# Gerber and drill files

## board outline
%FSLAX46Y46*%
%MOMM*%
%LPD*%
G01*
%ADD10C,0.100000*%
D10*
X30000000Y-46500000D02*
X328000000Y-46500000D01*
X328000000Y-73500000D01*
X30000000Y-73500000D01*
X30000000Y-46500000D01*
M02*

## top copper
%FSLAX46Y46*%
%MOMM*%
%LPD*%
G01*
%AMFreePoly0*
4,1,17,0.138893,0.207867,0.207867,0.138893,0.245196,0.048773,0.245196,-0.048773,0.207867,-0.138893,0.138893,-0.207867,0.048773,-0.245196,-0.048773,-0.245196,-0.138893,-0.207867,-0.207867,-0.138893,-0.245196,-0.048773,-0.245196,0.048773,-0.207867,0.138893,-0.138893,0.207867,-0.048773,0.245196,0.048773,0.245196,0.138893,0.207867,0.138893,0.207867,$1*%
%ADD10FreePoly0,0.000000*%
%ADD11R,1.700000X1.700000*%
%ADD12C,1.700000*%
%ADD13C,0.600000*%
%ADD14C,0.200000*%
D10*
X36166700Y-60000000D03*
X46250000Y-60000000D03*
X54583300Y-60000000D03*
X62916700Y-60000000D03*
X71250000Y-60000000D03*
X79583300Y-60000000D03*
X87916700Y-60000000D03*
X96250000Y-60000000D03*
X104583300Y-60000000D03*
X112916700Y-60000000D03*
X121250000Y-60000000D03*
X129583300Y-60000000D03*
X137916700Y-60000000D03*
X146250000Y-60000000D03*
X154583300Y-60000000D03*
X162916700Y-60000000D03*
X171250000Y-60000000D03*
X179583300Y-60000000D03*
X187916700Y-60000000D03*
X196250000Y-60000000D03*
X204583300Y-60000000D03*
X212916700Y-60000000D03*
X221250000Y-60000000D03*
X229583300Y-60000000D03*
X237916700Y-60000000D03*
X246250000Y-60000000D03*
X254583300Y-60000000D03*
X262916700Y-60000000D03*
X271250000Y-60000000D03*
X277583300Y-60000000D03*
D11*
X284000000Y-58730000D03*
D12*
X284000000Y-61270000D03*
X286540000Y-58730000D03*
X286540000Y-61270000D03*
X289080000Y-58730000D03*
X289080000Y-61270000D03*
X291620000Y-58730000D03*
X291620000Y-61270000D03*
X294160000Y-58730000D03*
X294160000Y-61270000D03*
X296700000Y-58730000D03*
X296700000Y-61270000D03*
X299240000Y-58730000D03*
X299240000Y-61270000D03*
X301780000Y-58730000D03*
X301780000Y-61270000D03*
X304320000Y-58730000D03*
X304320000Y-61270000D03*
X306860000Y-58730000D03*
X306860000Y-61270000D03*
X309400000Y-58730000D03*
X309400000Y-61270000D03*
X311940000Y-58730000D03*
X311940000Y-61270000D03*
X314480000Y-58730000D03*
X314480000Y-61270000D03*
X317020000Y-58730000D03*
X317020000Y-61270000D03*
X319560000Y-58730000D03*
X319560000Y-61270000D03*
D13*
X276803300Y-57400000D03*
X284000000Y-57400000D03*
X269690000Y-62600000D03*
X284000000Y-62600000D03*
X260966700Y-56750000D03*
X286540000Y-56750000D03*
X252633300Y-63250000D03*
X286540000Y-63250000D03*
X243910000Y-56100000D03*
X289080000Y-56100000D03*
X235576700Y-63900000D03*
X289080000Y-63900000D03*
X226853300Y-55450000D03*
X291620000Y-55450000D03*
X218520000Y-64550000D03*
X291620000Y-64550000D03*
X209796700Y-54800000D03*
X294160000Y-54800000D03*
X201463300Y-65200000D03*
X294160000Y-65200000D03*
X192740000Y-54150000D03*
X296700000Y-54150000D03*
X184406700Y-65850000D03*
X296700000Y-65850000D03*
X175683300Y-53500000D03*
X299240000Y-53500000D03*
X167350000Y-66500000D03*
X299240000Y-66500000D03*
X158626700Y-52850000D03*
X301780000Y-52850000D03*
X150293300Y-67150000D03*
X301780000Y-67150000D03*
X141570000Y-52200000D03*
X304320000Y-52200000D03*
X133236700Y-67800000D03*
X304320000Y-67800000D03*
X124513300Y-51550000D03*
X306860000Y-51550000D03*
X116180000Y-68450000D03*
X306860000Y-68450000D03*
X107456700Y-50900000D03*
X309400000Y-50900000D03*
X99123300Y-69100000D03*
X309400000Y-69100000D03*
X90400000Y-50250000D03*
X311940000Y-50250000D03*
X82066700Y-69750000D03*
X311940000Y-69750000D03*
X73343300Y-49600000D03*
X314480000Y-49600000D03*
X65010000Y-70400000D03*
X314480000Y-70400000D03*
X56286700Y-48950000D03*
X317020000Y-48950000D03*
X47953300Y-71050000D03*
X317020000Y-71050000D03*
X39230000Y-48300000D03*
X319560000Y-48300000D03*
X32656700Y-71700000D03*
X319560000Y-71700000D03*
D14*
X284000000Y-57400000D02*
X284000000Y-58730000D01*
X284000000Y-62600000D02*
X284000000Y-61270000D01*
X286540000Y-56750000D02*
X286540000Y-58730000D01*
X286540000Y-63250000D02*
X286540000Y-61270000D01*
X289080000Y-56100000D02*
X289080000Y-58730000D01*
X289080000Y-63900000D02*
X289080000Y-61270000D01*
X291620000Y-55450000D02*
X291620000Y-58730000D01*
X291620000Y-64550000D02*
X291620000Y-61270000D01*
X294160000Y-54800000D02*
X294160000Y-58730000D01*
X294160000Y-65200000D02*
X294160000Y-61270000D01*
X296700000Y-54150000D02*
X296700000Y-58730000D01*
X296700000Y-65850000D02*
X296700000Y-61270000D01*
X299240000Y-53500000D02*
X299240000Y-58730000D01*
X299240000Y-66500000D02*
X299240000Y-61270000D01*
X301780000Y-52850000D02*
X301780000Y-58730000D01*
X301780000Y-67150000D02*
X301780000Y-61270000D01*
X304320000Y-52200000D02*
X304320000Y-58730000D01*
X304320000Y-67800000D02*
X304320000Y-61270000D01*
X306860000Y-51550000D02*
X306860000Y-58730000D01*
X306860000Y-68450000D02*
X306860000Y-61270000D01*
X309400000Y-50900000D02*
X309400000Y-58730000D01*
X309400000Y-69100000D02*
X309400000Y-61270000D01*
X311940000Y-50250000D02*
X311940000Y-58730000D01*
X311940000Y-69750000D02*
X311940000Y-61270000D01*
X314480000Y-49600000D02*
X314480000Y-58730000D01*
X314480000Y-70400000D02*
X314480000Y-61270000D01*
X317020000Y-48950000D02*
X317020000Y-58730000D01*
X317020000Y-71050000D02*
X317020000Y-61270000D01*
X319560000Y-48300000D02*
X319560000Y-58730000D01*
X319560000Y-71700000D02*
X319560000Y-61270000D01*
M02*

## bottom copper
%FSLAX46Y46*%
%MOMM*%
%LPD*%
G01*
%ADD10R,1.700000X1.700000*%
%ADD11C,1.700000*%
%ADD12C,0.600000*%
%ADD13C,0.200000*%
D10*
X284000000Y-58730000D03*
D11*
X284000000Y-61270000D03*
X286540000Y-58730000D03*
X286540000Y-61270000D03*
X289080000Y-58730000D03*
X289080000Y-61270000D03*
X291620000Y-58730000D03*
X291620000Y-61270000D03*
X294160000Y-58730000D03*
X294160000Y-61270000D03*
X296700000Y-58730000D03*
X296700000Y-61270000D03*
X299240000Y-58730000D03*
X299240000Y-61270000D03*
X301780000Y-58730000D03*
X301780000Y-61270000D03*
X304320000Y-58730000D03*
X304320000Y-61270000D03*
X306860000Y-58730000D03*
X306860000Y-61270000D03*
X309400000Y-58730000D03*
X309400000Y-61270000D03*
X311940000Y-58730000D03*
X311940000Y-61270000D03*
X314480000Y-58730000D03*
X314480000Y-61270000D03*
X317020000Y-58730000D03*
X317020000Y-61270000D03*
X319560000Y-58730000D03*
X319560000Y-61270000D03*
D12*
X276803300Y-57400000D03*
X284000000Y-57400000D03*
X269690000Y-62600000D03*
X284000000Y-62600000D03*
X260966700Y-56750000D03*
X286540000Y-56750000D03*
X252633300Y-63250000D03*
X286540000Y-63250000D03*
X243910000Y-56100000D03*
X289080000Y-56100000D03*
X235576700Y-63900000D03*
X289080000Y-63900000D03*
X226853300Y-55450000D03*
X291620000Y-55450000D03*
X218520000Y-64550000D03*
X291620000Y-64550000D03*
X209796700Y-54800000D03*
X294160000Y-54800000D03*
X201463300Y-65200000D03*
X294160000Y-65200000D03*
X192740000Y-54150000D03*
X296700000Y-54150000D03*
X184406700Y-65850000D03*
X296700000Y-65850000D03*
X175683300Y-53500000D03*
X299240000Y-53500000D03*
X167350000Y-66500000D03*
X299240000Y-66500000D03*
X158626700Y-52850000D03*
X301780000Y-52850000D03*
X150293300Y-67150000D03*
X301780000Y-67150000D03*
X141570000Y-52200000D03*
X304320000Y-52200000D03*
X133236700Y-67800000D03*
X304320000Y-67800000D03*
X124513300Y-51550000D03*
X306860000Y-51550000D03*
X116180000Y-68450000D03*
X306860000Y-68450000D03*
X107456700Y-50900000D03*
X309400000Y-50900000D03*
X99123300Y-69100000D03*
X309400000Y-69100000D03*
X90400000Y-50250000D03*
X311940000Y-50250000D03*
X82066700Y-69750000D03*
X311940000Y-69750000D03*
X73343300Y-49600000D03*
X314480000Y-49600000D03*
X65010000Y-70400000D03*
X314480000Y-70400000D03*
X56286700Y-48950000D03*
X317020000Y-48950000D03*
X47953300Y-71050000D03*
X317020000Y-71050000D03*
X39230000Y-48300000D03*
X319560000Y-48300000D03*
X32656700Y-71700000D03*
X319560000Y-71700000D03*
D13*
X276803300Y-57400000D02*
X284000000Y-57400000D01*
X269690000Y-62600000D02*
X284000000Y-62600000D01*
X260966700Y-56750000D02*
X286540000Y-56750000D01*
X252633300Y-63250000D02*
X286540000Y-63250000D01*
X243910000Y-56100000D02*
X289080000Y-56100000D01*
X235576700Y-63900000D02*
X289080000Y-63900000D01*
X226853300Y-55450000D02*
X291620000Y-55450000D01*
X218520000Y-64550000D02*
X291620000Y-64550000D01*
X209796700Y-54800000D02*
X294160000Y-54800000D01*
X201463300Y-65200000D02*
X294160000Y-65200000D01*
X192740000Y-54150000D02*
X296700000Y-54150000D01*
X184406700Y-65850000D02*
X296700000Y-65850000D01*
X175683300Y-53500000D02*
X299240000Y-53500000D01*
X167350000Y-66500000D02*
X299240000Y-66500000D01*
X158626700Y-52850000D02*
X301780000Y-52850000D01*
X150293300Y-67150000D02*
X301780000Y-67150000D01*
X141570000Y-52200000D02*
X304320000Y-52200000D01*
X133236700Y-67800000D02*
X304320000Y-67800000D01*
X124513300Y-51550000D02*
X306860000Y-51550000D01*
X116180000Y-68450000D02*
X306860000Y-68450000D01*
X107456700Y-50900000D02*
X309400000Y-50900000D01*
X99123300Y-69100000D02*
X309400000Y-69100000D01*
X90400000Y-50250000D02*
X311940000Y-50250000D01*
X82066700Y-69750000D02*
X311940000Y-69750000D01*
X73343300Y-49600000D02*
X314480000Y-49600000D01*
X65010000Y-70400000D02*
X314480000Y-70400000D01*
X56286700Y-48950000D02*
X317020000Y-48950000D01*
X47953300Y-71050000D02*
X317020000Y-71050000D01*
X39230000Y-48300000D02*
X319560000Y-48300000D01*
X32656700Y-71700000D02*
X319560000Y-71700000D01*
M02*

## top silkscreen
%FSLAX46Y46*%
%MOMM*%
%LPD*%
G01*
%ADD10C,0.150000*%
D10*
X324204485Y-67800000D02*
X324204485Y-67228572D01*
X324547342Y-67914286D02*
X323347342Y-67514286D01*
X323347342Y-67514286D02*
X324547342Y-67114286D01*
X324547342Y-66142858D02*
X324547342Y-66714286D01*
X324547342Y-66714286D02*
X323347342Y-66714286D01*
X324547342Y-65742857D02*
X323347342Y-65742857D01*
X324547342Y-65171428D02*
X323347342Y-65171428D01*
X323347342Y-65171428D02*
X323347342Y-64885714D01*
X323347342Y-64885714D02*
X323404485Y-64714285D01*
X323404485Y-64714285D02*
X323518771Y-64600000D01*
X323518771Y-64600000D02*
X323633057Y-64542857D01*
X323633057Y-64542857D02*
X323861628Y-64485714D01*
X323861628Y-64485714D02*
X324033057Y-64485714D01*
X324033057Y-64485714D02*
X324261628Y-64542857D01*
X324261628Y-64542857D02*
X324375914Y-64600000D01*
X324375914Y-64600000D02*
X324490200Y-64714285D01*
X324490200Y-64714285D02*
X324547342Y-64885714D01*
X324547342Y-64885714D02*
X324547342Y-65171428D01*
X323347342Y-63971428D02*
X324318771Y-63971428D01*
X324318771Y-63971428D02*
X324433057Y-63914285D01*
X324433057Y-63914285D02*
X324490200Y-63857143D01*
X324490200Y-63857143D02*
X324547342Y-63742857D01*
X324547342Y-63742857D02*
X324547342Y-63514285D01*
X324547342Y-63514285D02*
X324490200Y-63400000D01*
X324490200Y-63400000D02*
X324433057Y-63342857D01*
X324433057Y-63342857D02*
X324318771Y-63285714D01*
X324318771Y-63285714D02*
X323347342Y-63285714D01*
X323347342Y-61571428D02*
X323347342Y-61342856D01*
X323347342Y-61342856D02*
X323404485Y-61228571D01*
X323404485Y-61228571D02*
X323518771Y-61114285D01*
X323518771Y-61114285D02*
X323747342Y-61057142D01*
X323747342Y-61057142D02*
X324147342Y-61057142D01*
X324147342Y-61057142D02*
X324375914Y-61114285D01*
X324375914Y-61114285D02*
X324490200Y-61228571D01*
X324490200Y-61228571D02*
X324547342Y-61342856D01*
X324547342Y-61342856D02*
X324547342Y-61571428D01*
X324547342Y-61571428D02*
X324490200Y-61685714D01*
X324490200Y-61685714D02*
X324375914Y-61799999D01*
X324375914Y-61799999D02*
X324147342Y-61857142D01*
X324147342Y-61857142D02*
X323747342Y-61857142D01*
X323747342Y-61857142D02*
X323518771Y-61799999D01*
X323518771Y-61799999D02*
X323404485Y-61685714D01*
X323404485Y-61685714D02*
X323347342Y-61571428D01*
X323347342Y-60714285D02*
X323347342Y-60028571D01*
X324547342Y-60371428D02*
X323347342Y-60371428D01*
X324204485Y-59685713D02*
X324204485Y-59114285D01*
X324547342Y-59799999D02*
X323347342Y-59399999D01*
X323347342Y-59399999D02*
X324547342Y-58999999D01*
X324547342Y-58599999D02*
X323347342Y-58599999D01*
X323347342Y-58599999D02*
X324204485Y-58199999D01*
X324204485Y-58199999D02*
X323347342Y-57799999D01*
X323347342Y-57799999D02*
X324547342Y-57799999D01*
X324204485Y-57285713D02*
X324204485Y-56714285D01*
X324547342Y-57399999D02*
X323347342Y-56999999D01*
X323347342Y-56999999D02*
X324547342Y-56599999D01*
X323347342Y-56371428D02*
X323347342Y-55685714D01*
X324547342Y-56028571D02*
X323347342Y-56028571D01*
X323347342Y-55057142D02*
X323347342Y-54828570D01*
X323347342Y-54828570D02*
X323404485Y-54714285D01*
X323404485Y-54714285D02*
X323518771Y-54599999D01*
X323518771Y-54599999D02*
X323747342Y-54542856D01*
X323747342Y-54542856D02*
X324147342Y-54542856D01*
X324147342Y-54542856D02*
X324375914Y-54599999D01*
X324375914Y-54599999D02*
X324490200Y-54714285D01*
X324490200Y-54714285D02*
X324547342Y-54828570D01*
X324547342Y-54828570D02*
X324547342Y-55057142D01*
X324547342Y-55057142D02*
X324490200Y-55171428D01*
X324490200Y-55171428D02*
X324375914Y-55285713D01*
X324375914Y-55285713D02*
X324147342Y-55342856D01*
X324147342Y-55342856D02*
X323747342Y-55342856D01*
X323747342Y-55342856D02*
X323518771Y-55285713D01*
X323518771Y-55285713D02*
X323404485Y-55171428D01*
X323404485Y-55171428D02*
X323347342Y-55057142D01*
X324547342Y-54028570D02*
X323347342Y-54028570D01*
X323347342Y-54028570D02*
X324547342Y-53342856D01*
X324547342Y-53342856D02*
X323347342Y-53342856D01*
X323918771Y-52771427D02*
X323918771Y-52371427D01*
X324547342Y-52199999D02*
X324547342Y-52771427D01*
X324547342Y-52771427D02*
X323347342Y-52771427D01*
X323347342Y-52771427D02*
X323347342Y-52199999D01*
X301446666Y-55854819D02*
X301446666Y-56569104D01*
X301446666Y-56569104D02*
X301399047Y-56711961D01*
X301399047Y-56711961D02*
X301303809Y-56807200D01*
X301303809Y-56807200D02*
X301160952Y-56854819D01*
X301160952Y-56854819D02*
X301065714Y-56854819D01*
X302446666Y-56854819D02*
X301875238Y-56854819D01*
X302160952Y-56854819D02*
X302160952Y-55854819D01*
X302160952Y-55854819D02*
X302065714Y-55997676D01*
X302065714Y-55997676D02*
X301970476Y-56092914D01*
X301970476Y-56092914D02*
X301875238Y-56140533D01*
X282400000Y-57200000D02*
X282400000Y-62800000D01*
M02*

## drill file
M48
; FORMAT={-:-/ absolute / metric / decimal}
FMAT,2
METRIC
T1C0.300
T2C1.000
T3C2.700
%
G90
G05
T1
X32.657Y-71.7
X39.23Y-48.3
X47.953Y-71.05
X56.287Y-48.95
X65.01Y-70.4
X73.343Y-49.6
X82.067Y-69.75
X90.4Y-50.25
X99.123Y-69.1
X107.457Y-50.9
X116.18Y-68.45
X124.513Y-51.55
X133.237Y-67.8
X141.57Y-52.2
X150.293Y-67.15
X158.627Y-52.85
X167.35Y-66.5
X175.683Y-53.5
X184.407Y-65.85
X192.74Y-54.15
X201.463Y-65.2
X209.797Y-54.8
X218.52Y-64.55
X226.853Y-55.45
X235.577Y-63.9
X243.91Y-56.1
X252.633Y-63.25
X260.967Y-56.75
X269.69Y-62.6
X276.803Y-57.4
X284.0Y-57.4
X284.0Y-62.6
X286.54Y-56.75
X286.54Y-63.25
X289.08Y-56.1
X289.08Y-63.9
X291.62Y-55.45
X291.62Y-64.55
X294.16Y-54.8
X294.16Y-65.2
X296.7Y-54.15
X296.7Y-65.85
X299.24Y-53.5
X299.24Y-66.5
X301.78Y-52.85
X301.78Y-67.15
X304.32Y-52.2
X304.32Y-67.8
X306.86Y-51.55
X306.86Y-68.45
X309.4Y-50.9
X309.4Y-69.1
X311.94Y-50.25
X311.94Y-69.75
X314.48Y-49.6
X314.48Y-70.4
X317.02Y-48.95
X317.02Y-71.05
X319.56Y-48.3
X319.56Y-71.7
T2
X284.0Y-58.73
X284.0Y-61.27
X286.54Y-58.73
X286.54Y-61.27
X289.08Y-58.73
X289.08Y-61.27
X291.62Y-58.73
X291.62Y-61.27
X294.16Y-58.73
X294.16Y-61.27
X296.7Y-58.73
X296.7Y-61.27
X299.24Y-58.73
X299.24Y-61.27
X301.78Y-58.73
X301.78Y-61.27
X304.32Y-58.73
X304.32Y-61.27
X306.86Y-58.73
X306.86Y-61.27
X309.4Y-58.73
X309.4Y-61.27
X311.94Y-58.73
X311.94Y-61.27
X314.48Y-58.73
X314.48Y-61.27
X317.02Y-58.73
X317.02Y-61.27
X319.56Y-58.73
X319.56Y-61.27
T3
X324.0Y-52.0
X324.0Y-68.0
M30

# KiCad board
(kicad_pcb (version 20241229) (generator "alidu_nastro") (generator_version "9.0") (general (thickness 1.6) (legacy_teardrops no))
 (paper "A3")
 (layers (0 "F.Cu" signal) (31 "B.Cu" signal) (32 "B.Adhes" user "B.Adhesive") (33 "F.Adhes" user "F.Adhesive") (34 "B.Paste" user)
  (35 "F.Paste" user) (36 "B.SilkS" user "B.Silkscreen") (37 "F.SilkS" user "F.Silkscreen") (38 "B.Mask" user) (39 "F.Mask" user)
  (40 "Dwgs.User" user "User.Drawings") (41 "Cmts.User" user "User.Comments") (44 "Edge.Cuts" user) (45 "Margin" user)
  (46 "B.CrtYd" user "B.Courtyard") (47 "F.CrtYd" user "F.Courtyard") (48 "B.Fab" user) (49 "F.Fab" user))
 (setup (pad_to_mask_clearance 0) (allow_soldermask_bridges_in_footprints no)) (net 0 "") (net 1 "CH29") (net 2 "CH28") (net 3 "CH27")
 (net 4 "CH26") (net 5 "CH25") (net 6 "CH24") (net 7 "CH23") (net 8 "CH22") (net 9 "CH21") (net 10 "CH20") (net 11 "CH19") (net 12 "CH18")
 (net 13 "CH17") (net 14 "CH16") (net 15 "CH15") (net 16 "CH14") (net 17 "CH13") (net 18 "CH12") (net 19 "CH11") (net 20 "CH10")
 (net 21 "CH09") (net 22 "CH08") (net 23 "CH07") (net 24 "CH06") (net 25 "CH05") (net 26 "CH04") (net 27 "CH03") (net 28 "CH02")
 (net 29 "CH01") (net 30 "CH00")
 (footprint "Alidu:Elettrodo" (layer "F.Cu") (at 36.1667 60.0)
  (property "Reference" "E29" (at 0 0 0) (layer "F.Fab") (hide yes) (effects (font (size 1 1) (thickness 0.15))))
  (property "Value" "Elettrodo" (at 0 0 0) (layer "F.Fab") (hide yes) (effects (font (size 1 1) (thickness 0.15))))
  (pad "1" smd custom (at 0 0) (size 0.5 0.5) (layers "F.Cu") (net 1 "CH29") (zone_connect 0) (options (clearance outline) (anchor circle))
   (primitives)))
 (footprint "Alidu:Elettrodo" (layer "F.Cu") (at 46.25 60.0)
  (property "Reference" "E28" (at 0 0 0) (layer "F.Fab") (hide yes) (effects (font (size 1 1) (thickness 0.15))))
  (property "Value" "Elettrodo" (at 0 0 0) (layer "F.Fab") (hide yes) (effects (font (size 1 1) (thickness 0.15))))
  (pad "1" smd custom (at 0 0) (size 0.5 0.5) (layers "F.Cu") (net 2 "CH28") (zone_connect 0) (options (clearance outline) (anchor circle))
   (primitives)))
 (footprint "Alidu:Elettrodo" (layer "F.Cu") (at 54.5833 60.0)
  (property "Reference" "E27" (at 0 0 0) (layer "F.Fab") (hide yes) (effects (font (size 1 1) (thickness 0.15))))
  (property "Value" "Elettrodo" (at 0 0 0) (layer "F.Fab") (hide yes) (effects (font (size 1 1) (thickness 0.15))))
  (pad "1" smd custom (at 0 0) (size 0.5 0.5) (layers "F.Cu") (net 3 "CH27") (zone_connect 0) (options (clearance outline) (anchor circle))
   (primitives)))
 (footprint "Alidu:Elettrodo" (layer "F.Cu") (at 62.9167 60.0)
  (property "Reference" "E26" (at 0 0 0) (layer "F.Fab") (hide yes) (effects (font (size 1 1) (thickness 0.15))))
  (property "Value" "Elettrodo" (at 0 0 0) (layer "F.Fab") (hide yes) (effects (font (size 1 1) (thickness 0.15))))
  (pad "1" smd custom (at 0 0) (size 0.5 0.5) (layers "F.Cu") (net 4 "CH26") (zone_connect 0) (options (clearance outline) (anchor circle))
   (primitives)))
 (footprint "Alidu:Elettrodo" (layer "F.Cu") (at 71.25 60.0)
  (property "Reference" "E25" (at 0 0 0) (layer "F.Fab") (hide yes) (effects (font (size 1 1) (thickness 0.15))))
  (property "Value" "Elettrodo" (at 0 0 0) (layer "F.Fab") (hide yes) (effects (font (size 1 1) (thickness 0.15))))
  (pad "1" smd custom (at 0 0) (size 0.5 0.5) (layers "F.Cu") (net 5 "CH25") (zone_connect 0) (options (clearance outline) (anchor circle))
   (primitives)))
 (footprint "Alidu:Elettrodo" (layer "F.Cu") (at 79.5833 60.0)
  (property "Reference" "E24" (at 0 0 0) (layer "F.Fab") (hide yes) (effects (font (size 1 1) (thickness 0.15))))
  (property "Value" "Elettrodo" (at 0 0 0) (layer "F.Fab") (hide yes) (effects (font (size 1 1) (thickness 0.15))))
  (pad "1" smd custom (at 0 0) (size 0.5 0.5) (layers "F.Cu") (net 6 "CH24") (zone_connect 0) (options (clearance outline) (anchor circle))
   (primitives)))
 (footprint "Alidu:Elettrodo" (layer "F.Cu") (at 87.9167 60.0)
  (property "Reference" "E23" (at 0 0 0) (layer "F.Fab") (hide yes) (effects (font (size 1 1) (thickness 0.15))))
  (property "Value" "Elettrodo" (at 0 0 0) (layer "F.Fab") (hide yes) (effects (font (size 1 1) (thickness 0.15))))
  (pad "1" smd custom (at 0 0) (size 0.5 0.5) (layers "F.Cu") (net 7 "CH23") (zone_connect 0) (options (clearance outline) (anchor circle))
   (primitives)))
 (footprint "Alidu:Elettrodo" (layer "F.Cu") (at 96.25 60.0)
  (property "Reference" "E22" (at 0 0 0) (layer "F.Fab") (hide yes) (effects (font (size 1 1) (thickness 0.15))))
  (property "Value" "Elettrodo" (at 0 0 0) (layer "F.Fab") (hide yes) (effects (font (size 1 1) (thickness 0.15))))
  (pad "1" smd custom (at 0 0) (size 0.5 0.5) (layers "F.Cu") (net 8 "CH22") (zone_connect 0) (options (clearance outline) (anchor circle))
   (primitives)))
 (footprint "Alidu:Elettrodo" (layer "F.Cu") (at 104.5833 60.0)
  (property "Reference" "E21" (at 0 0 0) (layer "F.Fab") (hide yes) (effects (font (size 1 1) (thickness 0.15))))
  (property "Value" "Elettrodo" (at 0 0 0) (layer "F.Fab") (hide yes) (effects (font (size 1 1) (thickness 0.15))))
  (pad "1" smd custom (at 0 0) (size 0.5 0.5) (layers "F.Cu") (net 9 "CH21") (zone_connect 0) (options (clearance outline) (anchor circle))
   (primitives)))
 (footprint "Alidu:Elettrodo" (layer "F.Cu") (at 112.9167 60.0)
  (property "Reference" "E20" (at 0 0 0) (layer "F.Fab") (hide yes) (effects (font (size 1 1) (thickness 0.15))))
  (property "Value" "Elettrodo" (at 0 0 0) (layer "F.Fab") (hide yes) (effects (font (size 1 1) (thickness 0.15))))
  (pad "1" smd custom (at 0 0) (size 0.5 0.5) (layers "F.Cu") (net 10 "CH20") (zone_connect 0) (options (clearance outline) (anchor circle))
   (primitives)))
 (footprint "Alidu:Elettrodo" (layer "F.Cu") (at 121.25 60.0)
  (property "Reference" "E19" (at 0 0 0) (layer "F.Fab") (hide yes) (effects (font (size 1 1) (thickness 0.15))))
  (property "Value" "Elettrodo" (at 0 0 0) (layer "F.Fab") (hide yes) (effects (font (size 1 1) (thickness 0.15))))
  (pad "1" smd custom (at 0 0) (size 0.5 0.5) (layers "F.Cu") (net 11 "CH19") (zone_connect 0) (options (clearance outline) (anchor circle))
   (primitives)))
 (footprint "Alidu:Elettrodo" (layer "F.Cu") (at 129.5833 60.0)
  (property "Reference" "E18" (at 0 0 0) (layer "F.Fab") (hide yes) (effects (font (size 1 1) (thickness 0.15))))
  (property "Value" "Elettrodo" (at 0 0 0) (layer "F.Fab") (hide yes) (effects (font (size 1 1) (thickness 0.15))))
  (pad "1" smd custom (at 0 0) (size 0.5 0.5) (layers "F.Cu") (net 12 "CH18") (zone_connect 0) (options (clearance outline) (anchor circle))
   (primitives)))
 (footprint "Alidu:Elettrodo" (layer "F.Cu") (at 137.9167 60.0)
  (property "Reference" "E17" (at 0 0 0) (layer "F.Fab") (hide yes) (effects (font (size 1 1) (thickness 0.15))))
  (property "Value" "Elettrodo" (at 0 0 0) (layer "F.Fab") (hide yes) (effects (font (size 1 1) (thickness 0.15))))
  (pad "1" smd custom (at 0 0) (size 0.5 0.5) (layers "F.Cu") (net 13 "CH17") (zone_connect 0) (options (clearance outline) (anchor circle))
   (primitives)))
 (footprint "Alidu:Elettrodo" (layer "F.Cu") (at 146.25 60.0)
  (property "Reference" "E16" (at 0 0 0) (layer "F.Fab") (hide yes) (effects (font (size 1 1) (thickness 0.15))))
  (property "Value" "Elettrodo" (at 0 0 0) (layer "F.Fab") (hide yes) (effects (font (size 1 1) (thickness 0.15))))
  (pad "1" smd custom (at 0 0) (size 0.5 0.5) (layers "F.Cu") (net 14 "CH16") (zone_connect 0) (options (clearance outline) (anchor circle))
   (primitives)))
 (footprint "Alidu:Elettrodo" (layer "F.Cu") (at 154.5833 60.0)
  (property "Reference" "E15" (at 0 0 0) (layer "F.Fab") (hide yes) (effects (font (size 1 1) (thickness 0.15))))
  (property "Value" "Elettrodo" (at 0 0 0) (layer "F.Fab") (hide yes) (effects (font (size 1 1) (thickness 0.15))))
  (pad "1" smd custom (at 0 0) (size 0.5 0.5) (layers "F.Cu") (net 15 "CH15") (zone_connect 0) (options (clearance outline) (anchor circle))
   (primitives)))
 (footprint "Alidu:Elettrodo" (layer "F.Cu") (at 162.9167 60.0)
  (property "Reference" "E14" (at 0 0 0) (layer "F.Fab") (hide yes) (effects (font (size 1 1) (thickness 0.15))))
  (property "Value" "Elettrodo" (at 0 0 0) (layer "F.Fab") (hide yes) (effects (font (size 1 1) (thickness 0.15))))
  (pad "1" smd custom (at 0 0) (size 0.5 0.5) (layers "F.Cu") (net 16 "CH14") (zone_connect 0) (options (clearance outline) (anchor circle))
   (primitives)))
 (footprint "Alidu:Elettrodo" (layer "F.Cu") (at 171.25 60.0)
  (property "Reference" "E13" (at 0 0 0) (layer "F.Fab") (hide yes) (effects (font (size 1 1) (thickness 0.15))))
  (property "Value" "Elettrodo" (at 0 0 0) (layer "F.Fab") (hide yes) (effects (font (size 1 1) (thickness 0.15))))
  (pad "1" smd custom (at 0 0) (size 0.5 0.5) (layers "F.Cu") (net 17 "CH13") (zone_connect 0) (options (clearance outline) (anchor circle))
   (primitives)))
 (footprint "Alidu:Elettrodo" (layer "F.Cu") (at 179.5833 60.0)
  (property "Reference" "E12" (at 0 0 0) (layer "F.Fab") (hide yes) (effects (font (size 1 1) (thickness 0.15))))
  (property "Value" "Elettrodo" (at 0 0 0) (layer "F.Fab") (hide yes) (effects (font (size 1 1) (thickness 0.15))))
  (pad "1" smd custom (at 0 0) (size 0.5 0.5) (layers "F.Cu") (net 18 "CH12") (zone_connect 0) (options (clearance outline) (anchor circle))
   (primitives)))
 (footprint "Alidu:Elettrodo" (layer "F.Cu") (at 187.9167 60.0)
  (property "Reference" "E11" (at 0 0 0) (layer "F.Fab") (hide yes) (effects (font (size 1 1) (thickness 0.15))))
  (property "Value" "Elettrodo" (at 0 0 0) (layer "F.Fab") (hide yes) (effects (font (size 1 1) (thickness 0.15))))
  (pad "1" smd custom (at 0 0) (size 0.5 0.5) (layers "F.Cu") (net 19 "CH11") (zone_connect 0) (options (clearance outline) (anchor circle))
   (primitives)))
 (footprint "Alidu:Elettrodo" (layer "F.Cu") (at 196.25 60.0)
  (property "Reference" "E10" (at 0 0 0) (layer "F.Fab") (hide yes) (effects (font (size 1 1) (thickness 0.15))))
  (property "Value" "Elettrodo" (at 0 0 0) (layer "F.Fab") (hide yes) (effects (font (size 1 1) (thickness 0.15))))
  (pad "1" smd custom (at 0 0) (size 0.5 0.5) (layers "F.Cu") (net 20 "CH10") (zone_connect 0) (options (clearance outline) (anchor circle))
   (primitives)))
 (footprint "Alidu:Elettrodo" (layer "F.Cu") (at 204.5833 60.0)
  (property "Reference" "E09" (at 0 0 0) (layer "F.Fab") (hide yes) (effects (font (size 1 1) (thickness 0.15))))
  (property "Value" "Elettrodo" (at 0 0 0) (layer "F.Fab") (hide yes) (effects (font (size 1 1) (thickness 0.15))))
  (pad "1" smd custom (at 0 0) (size 0.5 0.5) (layers "F.Cu") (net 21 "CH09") (zone_connect 0) (options (clearance outline) (anchor circle))
   (primitives)))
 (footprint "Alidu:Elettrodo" (layer "F.Cu") (at 212.9167 60.0)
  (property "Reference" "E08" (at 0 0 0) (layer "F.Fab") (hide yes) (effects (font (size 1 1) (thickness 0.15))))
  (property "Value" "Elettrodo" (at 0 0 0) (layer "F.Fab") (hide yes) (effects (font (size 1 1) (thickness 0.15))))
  (pad "1" smd custom (at 0 0) (size 0.5 0.5) (layers "F.Cu") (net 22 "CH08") (zone_connect 0) (options (clearance outline) (anchor circle))
   (primitives)))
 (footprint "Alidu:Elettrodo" (layer "F.Cu") (at 221.25 60.0)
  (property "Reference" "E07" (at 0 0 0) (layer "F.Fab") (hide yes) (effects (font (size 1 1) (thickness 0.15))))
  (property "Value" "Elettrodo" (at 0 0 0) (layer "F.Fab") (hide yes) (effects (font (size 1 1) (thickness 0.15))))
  (pad "1" smd custom (at 0 0) (size 0.5 0.5) (layers "F.Cu") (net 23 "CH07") (zone_connect 0) (options (clearance outline) (anchor circle))
   (primitives)))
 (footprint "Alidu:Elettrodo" (layer "F.Cu") (at 229.5833 60.0)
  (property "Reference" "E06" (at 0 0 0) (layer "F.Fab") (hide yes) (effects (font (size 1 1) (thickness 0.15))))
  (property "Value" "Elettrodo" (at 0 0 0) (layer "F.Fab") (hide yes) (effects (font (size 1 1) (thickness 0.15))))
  (pad "1" smd custom (at 0 0) (size 0.5 0.5) (layers "F.Cu") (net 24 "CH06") (zone_connect 0) (options (clearance outline) (anchor circle))
   (primitives)))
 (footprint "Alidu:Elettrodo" (layer "F.Cu") (at 237.9167 60.0)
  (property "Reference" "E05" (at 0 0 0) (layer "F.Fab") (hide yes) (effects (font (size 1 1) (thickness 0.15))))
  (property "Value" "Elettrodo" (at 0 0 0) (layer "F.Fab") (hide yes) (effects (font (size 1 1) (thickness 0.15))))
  (pad "1" smd custom (at 0 0) (size 0.5 0.5) (layers "F.Cu") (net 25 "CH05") (zone_connect 0) (options (clearance outline) (anchor circle))
   (primitives)))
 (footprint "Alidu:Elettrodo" (layer "F.Cu") (at 246.25 60.0)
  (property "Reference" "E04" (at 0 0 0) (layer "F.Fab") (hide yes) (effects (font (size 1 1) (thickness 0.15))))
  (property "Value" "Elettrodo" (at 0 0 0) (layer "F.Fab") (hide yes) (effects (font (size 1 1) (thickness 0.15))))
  (pad "1" smd custom (at 0 0) (size 0.5 0.5) (layers "F.Cu") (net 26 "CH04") (zone_connect 0) (options (clearance outline) (anchor circle))
   (primitives)))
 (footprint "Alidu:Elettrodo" (layer "F.Cu") (at 254.5833 60.0)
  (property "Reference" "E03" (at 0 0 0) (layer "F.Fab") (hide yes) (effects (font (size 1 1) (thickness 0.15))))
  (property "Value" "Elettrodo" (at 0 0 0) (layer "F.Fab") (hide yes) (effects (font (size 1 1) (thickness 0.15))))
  (pad "1" smd custom (at 0 0) (size 0.5 0.5) (layers "F.Cu") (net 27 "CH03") (zone_connect 0) (options (clearance outline) (anchor circle))
   (primitives)))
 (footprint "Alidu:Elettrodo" (layer "F.Cu") (at 262.9167 60.0)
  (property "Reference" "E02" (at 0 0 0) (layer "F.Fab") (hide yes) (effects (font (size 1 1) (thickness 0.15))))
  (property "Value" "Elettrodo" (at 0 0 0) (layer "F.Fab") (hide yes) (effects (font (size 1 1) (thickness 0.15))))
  (pad "1" smd custom (at 0 0) (size 0.5 0.5) (layers "F.Cu") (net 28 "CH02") (zone_connect 0) (options (clearance outline) (anchor circle))
   (primitives)))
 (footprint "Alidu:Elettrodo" (layer "F.Cu") (at 271.25 60.0)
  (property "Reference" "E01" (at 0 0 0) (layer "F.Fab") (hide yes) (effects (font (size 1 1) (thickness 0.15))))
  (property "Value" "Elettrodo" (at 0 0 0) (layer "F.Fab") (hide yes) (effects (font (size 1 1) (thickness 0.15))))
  (pad "1" smd custom (at 0 0) (size 0.5 0.5) (layers "F.Cu") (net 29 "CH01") (zone_connect 0) (options (clearance outline) (anchor circle))
   (primitives)))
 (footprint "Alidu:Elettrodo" (layer "F.Cu") (at 277.5833 60.0)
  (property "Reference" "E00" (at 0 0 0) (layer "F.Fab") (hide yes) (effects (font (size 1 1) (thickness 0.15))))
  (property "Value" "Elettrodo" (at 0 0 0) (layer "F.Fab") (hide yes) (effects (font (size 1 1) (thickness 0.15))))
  (pad "1" smd custom (at 0 0) (size 0.5 0.5) (layers "F.Cu") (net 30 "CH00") (zone_connect 0) (options (clearance outline) (anchor circle))
   (primitives)))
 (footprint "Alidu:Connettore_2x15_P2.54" (layer "F.Cu") (at 284.0 60.0)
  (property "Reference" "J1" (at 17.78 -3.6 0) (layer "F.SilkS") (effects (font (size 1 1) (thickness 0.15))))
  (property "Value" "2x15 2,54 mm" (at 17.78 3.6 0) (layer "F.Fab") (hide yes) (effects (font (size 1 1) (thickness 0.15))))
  (fp_line (start -1.6 -2.8) (end -1.6 2.8) (stroke (width 0.15) (type solid)) (layer "F.SilkS"))
  (pad "1" thru_hole rect (at 0.0 -1.27) (size 1.7 1.7) (drill 1.0) (layers "*.Cu" "*.Mask") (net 30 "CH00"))
  (pad "2" thru_hole circle (at 0.0 1.27) (size 1.7 1.7) (drill 1.0) (layers "*.Cu" "*.Mask") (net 29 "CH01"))
  (pad "3" thru_hole circle (at 2.54 -1.27) (size 1.7 1.7) (drill 1.0) (layers "*.Cu" "*.Mask") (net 28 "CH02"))
  (pad "4" thru_hole circle (at 2.54 1.27) (size 1.7 1.7) (drill 1.0) (layers "*.Cu" "*.Mask") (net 27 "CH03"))
  (pad "5" thru_hole circle (at 5.08 -1.27) (size 1.7 1.7) (drill 1.0) (layers "*.Cu" "*.Mask") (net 26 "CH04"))
  (pad "6" thru_hole circle (at 5.08 1.27) (size 1.7 1.7) (drill 1.0) (layers "*.Cu" "*.Mask") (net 25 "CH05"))
  (pad "7" thru_hole circle (at 7.62 -1.27) (size 1.7 1.7) (drill 1.0) (layers "*.Cu" "*.Mask") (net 24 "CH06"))
  (pad "8" thru_hole circle (at 7.62 1.27) (size 1.7 1.7) (drill 1.0) (layers "*.Cu" "*.Mask") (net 23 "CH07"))
  (pad "9" thru_hole circle (at 10.16 -1.27) (size 1.7 1.7) (drill 1.0) (layers "*.Cu" "*.Mask") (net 22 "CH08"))
  (pad "10" thru_hole circle (at 10.16 1.27) (size 1.7 1.7) (drill 1.0) (layers "*.Cu" "*.Mask") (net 21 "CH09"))
  (pad "11" thru_hole circle (at 12.7 -1.27) (size 1.7 1.7) (drill 1.0) (layers "*.Cu" "*.Mask") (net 20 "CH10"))
  (pad "12" thru_hole circle (at 12.7 1.27) (size 1.7 1.7) (drill 1.0) (layers "*.Cu" "*.Mask") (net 19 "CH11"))
  (pad "13" thru_hole circle (at 15.24 -1.27) (size 1.7 1.7) (drill 1.0) (layers "*.Cu" "*.Mask") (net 18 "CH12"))
  (pad "14" thru_hole circle (at 15.24 1.27) (size 1.7 1.7) (drill 1.0) (layers "*.Cu" "*.Mask") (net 17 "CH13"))
  (pad "15" thru_hole circle (at 17.78 -1.27) (size 1.7 1.7) (drill 1.0) (layers "*.Cu" "*.Mask") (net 16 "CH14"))
  (pad "16" thru_hole circle (at 17.78 1.27) (size 1.7 1.7) (drill 1.0) (layers "*.Cu" "*.Mask") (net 15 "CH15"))
  (pad "17" thru_hole circle (at 20.32 -1.27) (size 1.7 1.7) (drill 1.0) (layers "*.Cu" "*.Mask") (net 14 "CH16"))
  (pad "18" thru_hole circle (at 20.32 1.27) (size 1.7 1.7) (drill 1.0) (layers "*.Cu" "*.Mask") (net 13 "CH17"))
  (pad "19" thru_hole circle (at 22.86 -1.27) (size 1.7 1.7) (drill 1.0) (layers "*.Cu" "*.Mask") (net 12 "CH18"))
  (pad "20" thru_hole circle (at 22.86 1.27) (size 1.7 1.7) (drill 1.0) (layers "*.Cu" "*.Mask") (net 11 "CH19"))
  (pad "21" thru_hole circle (at 25.4 -1.27) (size 1.7 1.7) (drill 1.0) (layers "*.Cu" "*.Mask") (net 10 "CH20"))
  (pad "22" thru_hole circle (at 25.4 1.27) (size 1.7 1.7) (drill 1.0) (layers "*.Cu" "*.Mask") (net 9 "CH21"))
  (pad "23" thru_hole circle (at 27.94 -1.27) (size 1.7 1.7) (drill 1.0) (layers "*.Cu" "*.Mask") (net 8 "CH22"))
  (pad "24" thru_hole circle (at 27.94 1.27) (size 1.7 1.7) (drill 1.0) (layers "*.Cu" "*.Mask") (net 7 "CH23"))
  (pad "25" thru_hole circle (at 30.48 -1.27) (size 1.7 1.7) (drill 1.0) (layers "*.Cu" "*.Mask") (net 6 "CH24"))
  (pad "26" thru_hole circle (at 30.48 1.27) (size 1.7 1.7) (drill 1.0) (layers "*.Cu" "*.Mask") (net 5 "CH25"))
  (pad "27" thru_hole circle (at 33.02 -1.27) (size 1.7 1.7) (drill 1.0) (layers "*.Cu" "*.Mask") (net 4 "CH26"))
  (pad "28" thru_hole circle (at 33.02 1.27) (size 1.7 1.7) (drill 1.0) (layers "*.Cu" "*.Mask") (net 3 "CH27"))
  (pad "29" thru_hole circle (at 35.56 -1.27) (size 1.7 1.7) (drill 1.0) (layers "*.Cu" "*.Mask") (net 2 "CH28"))
  (pad "30" thru_hole circle (at 35.56 1.27) (size 1.7 1.7) (drill 1.0) (layers "*.Cu" "*.Mask") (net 1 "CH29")))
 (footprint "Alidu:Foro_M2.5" (layer "F.Cu") (at 324.0 52.0)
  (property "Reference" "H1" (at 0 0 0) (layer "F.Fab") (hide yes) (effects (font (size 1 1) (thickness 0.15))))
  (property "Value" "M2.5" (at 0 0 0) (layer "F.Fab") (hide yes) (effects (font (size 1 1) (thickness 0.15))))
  (pad "" np_thru_hole circle (at 0 0) (size 2.7 2.7) (drill 2.7) (layers "*.Cu" "*.Mask")))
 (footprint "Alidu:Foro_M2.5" (layer "F.Cu") (at 324.0 68.0)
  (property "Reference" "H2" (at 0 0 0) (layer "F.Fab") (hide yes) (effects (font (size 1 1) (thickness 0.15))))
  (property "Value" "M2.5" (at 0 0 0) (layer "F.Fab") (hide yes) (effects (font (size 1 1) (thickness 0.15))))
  (pad "" np_thru_hole circle (at 0 0) (size 2.7 2.7) (drill 2.7) (layers "*.Cu" "*.Mask")))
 (via (at 276.8033 57.4) (size 0.6) (drill 0.3) (layers "F.Cu" "B.Cu") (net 30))
 (segment (start 276.8033 57.4) (end 284.0 57.4) (width 0.2) (layer "B.Cu") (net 30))
 (via (at 284.0 57.4) (size 0.6) (drill 0.3) (layers "F.Cu" "B.Cu") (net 30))
 (segment (start 284.0 57.4) (end 284.0 58.73) (width 0.2) (layer "F.Cu") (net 30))
 (via (at 269.69 62.6) (size 0.6) (drill 0.3) (layers "F.Cu" "B.Cu") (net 29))
 (segment (start 269.69 62.6) (end 284.0 62.6) (width 0.2) (layer "B.Cu") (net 29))
 (via (at 284.0 62.6) (size 0.6) (drill 0.3) (layers "F.Cu" "B.Cu") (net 29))
 (segment (start 284.0 62.6) (end 284.0 61.27) (width 0.2) (layer "F.Cu") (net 29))
 (via (at 260.9667 56.75) (size 0.6) (drill 0.3) (layers "F.Cu" "B.Cu") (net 28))
 (segment (start 260.9667 56.75) (end 286.54 56.75) (width 0.2) (layer "B.Cu") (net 28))
 (via (at 286.54 56.75) (size 0.6) (drill 0.3) (layers "F.Cu" "B.Cu") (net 28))
 (segment (start 286.54 56.75) (end 286.54 58.73) (width 0.2) (layer "F.Cu") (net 28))
 (via (at 252.6333 63.25) (size 0.6) (drill 0.3) (layers "F.Cu" "B.Cu") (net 27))
 (segment (start 252.6333 63.25) (end 286.54 63.25) (width 0.2) (layer "B.Cu") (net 27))
 (via (at 286.54 63.25) (size 0.6) (drill 0.3) (layers "F.Cu" "B.Cu") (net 27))
 (segment (start 286.54 63.25) (end 286.54 61.27) (width 0.2) (layer "F.Cu") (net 27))
 (via (at 243.91 56.1) (size 0.6) (drill 0.3) (layers "F.Cu" "B.Cu") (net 26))
 (segment (start 243.91 56.1) (end 289.08 56.1) (width 0.2) (layer "B.Cu") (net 26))
 (via (at 289.08 56.1) (size 0.6) (drill 0.3) (layers "F.Cu" "B.Cu") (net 26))
 (segment (start 289.08 56.1) (end 289.08 58.73) (width 0.2) (layer "F.Cu") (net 26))
 (via (at 235.5767 63.9) (size 0.6) (drill 0.3) (layers "F.Cu" "B.Cu") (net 25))
 (segment (start 235.5767 63.9) (end 289.08 63.9) (width 0.2) (layer "B.Cu") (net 25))
 (via (at 289.08 63.9) (size 0.6) (drill 0.3) (layers "F.Cu" "B.Cu") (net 25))
 (segment (start 289.08 63.9) (end 289.08 61.27) (width 0.2) (layer "F.Cu") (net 25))
 (via (at 226.8533 55.45) (size 0.6) (drill 0.3) (layers "F.Cu" "B.Cu") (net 24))
 (segment (start 226.8533 55.45) (end 291.62 55.45) (width 0.2) (layer "B.Cu") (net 24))
 (via (at 291.62 55.45) (size 0.6) (drill 0.3) (layers "F.Cu" "B.Cu") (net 24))
 (segment (start 291.62 55.45) (end 291.62 58.73) (width 0.2) (layer "F.Cu") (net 24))
 (via (at 218.52 64.55) (size 0.6) (drill 0.3) (layers "F.Cu" "B.Cu") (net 23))
 (segment (start 218.52 64.55) (end 291.62 64.55) (width 0.2) (layer "B.Cu") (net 23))
 (via (at 291.62 64.55) (size 0.6) (drill 0.3) (layers "F.Cu" "B.Cu") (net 23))
 (segment (start 291.62 64.55) (end 291.62 61.27) (width 0.2) (layer "F.Cu") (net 23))
 (via (at 209.7967 54.8) (size 0.6) (drill 0.3) (layers "F.Cu" "B.Cu") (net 22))
 (segment (start 209.7967 54.8) (end 294.16 54.8) (width 0.2) (layer "B.Cu") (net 22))
 (via (at 294.16 54.8) (size 0.6) (drill 0.3) (layers "F.Cu" "B.Cu") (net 22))
 (segment (start 294.16 54.8) (end 294.16 58.73) (width 0.2) (layer "F.Cu") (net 22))
 (via (at 201.4633 65.2) (size 0.6) (drill 0.3) (layers "F.Cu" "B.Cu") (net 21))
 (segment (start 201.4633 65.2) (end 294.16 65.2) (width 0.2) (layer "B.Cu") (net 21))
 (via (at 294.16 65.2) (size 0.6) (drill 0.3) (layers "F.Cu" "B.Cu") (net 21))
 (segment (start 294.16 65.2) (end 294.16 61.27) (width 0.2) (layer "F.Cu") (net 21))
 (via (at 192.74 54.15) (size 0.6) (drill 0.3) (layers "F.Cu" "B.Cu") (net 20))
 (segment (start 192.74 54.15) (end 296.7 54.15) (width 0.2) (layer "B.Cu") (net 20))
 (via (at 296.7 54.15) (size 0.6) (drill 0.3) (layers "F.Cu" "B.Cu") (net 20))
 (segment (start 296.7 54.15) (end 296.7 58.73) (width 0.2) (layer "F.Cu") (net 20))
 (via (at 184.4067 65.85) (size 0.6) (drill 0.3) (layers "F.Cu" "B.Cu") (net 19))
 (segment (start 184.4067 65.85) (end 296.7 65.85) (width 0.2) (layer "B.Cu") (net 19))
 (via (at 296.7 65.85) (size 0.6) (drill 0.3) (layers "F.Cu" "B.Cu") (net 19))
 (segment (start 296.7 65.85) (end 296.7 61.27) (width 0.2) (layer "F.Cu") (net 19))
 (via (at 175.6833 53.5) (size 0.6) (drill 0.3) (layers "F.Cu" "B.Cu") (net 18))
 (segment (start 175.6833 53.5) (end 299.24 53.5) (width 0.2) (layer "B.Cu") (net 18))
 (via (at 299.24 53.5) (size 0.6) (drill 0.3) (layers "F.Cu" "B.Cu") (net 18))
 (segment (start 299.24 53.5) (end 299.24 58.73) (width 0.2) (layer "F.Cu") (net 18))
 (via (at 167.35 66.5) (size 0.6) (drill 0.3) (layers "F.Cu" "B.Cu") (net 17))
 (segment (start 167.35 66.5) (end 299.24 66.5) (width 0.2) (layer "B.Cu") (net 17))
 (via (at 299.24 66.5) (size 0.6) (drill 0.3) (layers "F.Cu" "B.Cu") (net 17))
 (segment (start 299.24 66.5) (end 299.24 61.27) (width 0.2) (layer "F.Cu") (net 17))
 (via (at 158.6267 52.85) (size 0.6) (drill 0.3) (layers "F.Cu" "B.Cu") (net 16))
 (segment (start 158.6267 52.85) (end 301.78 52.85) (width 0.2) (layer "B.Cu") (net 16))
 (via (at 301.78 52.85) (size 0.6) (drill 0.3) (layers "F.Cu" "B.Cu") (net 16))
 (segment (start 301.78 52.85) (end 301.78 58.73) (width 0.2) (layer "F.Cu") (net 16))
 (via (at 150.2933 67.15) (size 0.6) (drill 0.3) (layers "F.Cu" "B.Cu") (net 15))
 (segment (start 150.2933 67.15) (end 301.78 67.15) (width 0.2) (layer "B.Cu") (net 15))
 (via (at 301.78 67.15) (size 0.6) (drill 0.3) (layers "F.Cu" "B.Cu") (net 15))
 (segment (start 301.78 67.15) (end 301.78 61.27) (width 0.2) (layer "F.Cu") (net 15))
 (via (at 141.57 52.2) (size 0.6) (drill 0.3) (layers "F.Cu" "B.Cu") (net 14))
 (segment (start 141.57 52.2) (end 304.32 52.2) (width 0.2) (layer "B.Cu") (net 14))
 (via (at 304.32 52.2) (size 0.6) (drill 0.3) (layers "F.Cu" "B.Cu") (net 14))
 (segment (start 304.32 52.2) (end 304.32 58.73) (width 0.2) (layer "F.Cu") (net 14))
 (via (at 133.2367 67.8) (size 0.6) (drill 0.3) (layers "F.Cu" "B.Cu") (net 13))
 (segment (start 133.2367 67.8) (end 304.32 67.8) (width 0.2) (layer "B.Cu") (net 13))
 (via (at 304.32 67.8) (size 0.6) (drill 0.3) (layers "F.Cu" "B.Cu") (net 13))
 (segment (start 304.32 67.8) (end 304.32 61.27) (width 0.2) (layer "F.Cu") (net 13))
 (via (at 124.5133 51.55) (size 0.6) (drill 0.3) (layers "F.Cu" "B.Cu") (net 12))
 (segment (start 124.5133 51.55) (end 306.86 51.55) (width 0.2) (layer "B.Cu") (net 12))
 (via (at 306.86 51.55) (size 0.6) (drill 0.3) (layers "F.Cu" "B.Cu") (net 12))
 (segment (start 306.86 51.55) (end 306.86 58.73) (width 0.2) (layer "F.Cu") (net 12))
 (via (at 116.18 68.45) (size 0.6) (drill 0.3) (layers "F.Cu" "B.Cu") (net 11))
 (segment (start 116.18 68.45) (end 306.86 68.45) (width 0.2) (layer "B.Cu") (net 11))
 (via (at 306.86 68.45) (size 0.6) (drill 0.3) (layers "F.Cu" "B.Cu") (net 11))
 (segment (start 306.86 68.45) (end 306.86 61.27) (width 0.2) (layer "F.Cu") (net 11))
 (via (at 107.4567 50.9) (size 0.6) (drill 0.3) (layers "F.Cu" "B.Cu") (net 10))
 (segment (start 107.4567 50.9) (end 309.4 50.9) (width 0.2) (layer "B.Cu") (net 10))
 (via (at 309.4 50.9) (size 0.6) (drill 0.3) (layers "F.Cu" "B.Cu") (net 10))
 (segment (start 309.4 50.9) (end 309.4 58.73) (width 0.2) (layer "F.Cu") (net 10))
 (via (at 99.1233 69.1) (size 0.6) (drill 0.3) (layers "F.Cu" "B.Cu") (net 9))
 (segment (start 99.1233 69.1) (end 309.4 69.1) (width 0.2) (layer "B.Cu") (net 9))
 (via (at 309.4 69.1) (size 0.6) (drill 0.3) (layers "F.Cu" "B.Cu") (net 9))
 (segment (start 309.4 69.1) (end 309.4 61.27) (width 0.2) (layer "F.Cu") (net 9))
 (via (at 90.4 50.25) (size 0.6) (drill 0.3) (layers "F.Cu" "B.Cu") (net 8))
 (segment (start 90.4 50.25) (end 311.94 50.25) (width 0.2) (layer "B.Cu") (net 8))
 (via (at 311.94 50.25) (size 0.6) (drill 0.3) (layers "F.Cu" "B.Cu") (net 8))
 (segment (start 311.94 50.25) (end 311.94 58.73) (width 0.2) (layer "F.Cu") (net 8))
 (via (at 82.0667 69.75) (size 0.6) (drill 0.3) (layers "F.Cu" "B.Cu") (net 7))
 (segment (start 82.0667 69.75) (end 311.94 69.75) (width 0.2) (layer "B.Cu") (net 7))
 (via (at 311.94 69.75) (size 0.6) (drill 0.3) (layers "F.Cu" "B.Cu") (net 7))
 (segment (start 311.94 69.75) (end 311.94 61.27) (width 0.2) (layer "F.Cu") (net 7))
 (via (at 73.3433 49.6) (size 0.6) (drill 0.3) (layers "F.Cu" "B.Cu") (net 6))
 (segment (start 73.3433 49.6) (end 314.48 49.6) (width 0.2) (layer "B.Cu") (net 6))
 (via (at 314.48 49.6) (size 0.6) (drill 0.3) (layers "F.Cu" "B.Cu") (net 6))
 (segment (start 314.48 49.6) (end 314.48 58.73) (width 0.2) (layer "F.Cu") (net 6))
 (via (at 65.01 70.4) (size 0.6) (drill 0.3) (layers "F.Cu" "B.Cu") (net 5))
 (segment (start 65.01 70.4) (end 314.48 70.4) (width 0.2) (layer "B.Cu") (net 5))
 (via (at 314.48 70.4) (size 0.6) (drill 0.3) (layers "F.Cu" "B.Cu") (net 5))
 (segment (start 314.48 70.4) (end 314.48 61.27) (width 0.2) (layer "F.Cu") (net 5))
 (via (at 56.2867 48.95) (size 0.6) (drill 0.3) (layers "F.Cu" "B.Cu") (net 4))
 (segment (start 56.2867 48.95) (end 317.02 48.95) (width 0.2) (layer "B.Cu") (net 4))
 (via (at 317.02 48.95) (size 0.6) (drill 0.3) (layers "F.Cu" "B.Cu") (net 4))
 (segment (start 317.02 48.95) (end 317.02 58.73) (width 0.2) (layer "F.Cu") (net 4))
 (via (at 47.9533 71.05) (size 0.6) (drill 0.3) (layers "F.Cu" "B.Cu") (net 3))
 (segment (start 47.9533 71.05) (end 317.02 71.05) (width 0.2) (layer "B.Cu") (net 3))
 (via (at 317.02 71.05) (size 0.6) (drill 0.3) (layers "F.Cu" "B.Cu") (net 3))
 (segment (start 317.02 71.05) (end 317.02 61.27) (width 0.2) (layer "F.Cu") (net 3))
 (via (at 39.23 48.3) (size 0.6) (drill 0.3) (layers "F.Cu" "B.Cu") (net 2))
 (segment (start 39.23 48.3) (end 319.56 48.3) (width 0.2) (layer "B.Cu") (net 2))
 (via (at 319.56 48.3) (size 0.6) (drill 0.3) (layers "F.Cu" "B.Cu") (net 2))
 (segment (start 319.56 48.3) (end 319.56 58.73) (width 0.2) (layer "F.Cu") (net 2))
 (via (at 32.6567 71.7) (size 0.6) (drill 0.3) (layers "F.Cu" "B.Cu") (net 1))
 (segment (start 32.6567 71.7) (end 319.56 71.7) (width 0.2) (layer "B.Cu") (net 1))
 (via (at 319.56 71.7) (size 0.6) (drill 0.3) (layers "F.Cu" "B.Cu") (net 1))
 (segment (start 319.56 71.7) (end 319.56 61.27) (width 0.2) (layer "F.Cu") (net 1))
 (gr_rect (start 30.0 46.5) (end 328.0 73.5) (stroke (width 0.1) (type default)) (fill no) (layer "Edge.Cuts"))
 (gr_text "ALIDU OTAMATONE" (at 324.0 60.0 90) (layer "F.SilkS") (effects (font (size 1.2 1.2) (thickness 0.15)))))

